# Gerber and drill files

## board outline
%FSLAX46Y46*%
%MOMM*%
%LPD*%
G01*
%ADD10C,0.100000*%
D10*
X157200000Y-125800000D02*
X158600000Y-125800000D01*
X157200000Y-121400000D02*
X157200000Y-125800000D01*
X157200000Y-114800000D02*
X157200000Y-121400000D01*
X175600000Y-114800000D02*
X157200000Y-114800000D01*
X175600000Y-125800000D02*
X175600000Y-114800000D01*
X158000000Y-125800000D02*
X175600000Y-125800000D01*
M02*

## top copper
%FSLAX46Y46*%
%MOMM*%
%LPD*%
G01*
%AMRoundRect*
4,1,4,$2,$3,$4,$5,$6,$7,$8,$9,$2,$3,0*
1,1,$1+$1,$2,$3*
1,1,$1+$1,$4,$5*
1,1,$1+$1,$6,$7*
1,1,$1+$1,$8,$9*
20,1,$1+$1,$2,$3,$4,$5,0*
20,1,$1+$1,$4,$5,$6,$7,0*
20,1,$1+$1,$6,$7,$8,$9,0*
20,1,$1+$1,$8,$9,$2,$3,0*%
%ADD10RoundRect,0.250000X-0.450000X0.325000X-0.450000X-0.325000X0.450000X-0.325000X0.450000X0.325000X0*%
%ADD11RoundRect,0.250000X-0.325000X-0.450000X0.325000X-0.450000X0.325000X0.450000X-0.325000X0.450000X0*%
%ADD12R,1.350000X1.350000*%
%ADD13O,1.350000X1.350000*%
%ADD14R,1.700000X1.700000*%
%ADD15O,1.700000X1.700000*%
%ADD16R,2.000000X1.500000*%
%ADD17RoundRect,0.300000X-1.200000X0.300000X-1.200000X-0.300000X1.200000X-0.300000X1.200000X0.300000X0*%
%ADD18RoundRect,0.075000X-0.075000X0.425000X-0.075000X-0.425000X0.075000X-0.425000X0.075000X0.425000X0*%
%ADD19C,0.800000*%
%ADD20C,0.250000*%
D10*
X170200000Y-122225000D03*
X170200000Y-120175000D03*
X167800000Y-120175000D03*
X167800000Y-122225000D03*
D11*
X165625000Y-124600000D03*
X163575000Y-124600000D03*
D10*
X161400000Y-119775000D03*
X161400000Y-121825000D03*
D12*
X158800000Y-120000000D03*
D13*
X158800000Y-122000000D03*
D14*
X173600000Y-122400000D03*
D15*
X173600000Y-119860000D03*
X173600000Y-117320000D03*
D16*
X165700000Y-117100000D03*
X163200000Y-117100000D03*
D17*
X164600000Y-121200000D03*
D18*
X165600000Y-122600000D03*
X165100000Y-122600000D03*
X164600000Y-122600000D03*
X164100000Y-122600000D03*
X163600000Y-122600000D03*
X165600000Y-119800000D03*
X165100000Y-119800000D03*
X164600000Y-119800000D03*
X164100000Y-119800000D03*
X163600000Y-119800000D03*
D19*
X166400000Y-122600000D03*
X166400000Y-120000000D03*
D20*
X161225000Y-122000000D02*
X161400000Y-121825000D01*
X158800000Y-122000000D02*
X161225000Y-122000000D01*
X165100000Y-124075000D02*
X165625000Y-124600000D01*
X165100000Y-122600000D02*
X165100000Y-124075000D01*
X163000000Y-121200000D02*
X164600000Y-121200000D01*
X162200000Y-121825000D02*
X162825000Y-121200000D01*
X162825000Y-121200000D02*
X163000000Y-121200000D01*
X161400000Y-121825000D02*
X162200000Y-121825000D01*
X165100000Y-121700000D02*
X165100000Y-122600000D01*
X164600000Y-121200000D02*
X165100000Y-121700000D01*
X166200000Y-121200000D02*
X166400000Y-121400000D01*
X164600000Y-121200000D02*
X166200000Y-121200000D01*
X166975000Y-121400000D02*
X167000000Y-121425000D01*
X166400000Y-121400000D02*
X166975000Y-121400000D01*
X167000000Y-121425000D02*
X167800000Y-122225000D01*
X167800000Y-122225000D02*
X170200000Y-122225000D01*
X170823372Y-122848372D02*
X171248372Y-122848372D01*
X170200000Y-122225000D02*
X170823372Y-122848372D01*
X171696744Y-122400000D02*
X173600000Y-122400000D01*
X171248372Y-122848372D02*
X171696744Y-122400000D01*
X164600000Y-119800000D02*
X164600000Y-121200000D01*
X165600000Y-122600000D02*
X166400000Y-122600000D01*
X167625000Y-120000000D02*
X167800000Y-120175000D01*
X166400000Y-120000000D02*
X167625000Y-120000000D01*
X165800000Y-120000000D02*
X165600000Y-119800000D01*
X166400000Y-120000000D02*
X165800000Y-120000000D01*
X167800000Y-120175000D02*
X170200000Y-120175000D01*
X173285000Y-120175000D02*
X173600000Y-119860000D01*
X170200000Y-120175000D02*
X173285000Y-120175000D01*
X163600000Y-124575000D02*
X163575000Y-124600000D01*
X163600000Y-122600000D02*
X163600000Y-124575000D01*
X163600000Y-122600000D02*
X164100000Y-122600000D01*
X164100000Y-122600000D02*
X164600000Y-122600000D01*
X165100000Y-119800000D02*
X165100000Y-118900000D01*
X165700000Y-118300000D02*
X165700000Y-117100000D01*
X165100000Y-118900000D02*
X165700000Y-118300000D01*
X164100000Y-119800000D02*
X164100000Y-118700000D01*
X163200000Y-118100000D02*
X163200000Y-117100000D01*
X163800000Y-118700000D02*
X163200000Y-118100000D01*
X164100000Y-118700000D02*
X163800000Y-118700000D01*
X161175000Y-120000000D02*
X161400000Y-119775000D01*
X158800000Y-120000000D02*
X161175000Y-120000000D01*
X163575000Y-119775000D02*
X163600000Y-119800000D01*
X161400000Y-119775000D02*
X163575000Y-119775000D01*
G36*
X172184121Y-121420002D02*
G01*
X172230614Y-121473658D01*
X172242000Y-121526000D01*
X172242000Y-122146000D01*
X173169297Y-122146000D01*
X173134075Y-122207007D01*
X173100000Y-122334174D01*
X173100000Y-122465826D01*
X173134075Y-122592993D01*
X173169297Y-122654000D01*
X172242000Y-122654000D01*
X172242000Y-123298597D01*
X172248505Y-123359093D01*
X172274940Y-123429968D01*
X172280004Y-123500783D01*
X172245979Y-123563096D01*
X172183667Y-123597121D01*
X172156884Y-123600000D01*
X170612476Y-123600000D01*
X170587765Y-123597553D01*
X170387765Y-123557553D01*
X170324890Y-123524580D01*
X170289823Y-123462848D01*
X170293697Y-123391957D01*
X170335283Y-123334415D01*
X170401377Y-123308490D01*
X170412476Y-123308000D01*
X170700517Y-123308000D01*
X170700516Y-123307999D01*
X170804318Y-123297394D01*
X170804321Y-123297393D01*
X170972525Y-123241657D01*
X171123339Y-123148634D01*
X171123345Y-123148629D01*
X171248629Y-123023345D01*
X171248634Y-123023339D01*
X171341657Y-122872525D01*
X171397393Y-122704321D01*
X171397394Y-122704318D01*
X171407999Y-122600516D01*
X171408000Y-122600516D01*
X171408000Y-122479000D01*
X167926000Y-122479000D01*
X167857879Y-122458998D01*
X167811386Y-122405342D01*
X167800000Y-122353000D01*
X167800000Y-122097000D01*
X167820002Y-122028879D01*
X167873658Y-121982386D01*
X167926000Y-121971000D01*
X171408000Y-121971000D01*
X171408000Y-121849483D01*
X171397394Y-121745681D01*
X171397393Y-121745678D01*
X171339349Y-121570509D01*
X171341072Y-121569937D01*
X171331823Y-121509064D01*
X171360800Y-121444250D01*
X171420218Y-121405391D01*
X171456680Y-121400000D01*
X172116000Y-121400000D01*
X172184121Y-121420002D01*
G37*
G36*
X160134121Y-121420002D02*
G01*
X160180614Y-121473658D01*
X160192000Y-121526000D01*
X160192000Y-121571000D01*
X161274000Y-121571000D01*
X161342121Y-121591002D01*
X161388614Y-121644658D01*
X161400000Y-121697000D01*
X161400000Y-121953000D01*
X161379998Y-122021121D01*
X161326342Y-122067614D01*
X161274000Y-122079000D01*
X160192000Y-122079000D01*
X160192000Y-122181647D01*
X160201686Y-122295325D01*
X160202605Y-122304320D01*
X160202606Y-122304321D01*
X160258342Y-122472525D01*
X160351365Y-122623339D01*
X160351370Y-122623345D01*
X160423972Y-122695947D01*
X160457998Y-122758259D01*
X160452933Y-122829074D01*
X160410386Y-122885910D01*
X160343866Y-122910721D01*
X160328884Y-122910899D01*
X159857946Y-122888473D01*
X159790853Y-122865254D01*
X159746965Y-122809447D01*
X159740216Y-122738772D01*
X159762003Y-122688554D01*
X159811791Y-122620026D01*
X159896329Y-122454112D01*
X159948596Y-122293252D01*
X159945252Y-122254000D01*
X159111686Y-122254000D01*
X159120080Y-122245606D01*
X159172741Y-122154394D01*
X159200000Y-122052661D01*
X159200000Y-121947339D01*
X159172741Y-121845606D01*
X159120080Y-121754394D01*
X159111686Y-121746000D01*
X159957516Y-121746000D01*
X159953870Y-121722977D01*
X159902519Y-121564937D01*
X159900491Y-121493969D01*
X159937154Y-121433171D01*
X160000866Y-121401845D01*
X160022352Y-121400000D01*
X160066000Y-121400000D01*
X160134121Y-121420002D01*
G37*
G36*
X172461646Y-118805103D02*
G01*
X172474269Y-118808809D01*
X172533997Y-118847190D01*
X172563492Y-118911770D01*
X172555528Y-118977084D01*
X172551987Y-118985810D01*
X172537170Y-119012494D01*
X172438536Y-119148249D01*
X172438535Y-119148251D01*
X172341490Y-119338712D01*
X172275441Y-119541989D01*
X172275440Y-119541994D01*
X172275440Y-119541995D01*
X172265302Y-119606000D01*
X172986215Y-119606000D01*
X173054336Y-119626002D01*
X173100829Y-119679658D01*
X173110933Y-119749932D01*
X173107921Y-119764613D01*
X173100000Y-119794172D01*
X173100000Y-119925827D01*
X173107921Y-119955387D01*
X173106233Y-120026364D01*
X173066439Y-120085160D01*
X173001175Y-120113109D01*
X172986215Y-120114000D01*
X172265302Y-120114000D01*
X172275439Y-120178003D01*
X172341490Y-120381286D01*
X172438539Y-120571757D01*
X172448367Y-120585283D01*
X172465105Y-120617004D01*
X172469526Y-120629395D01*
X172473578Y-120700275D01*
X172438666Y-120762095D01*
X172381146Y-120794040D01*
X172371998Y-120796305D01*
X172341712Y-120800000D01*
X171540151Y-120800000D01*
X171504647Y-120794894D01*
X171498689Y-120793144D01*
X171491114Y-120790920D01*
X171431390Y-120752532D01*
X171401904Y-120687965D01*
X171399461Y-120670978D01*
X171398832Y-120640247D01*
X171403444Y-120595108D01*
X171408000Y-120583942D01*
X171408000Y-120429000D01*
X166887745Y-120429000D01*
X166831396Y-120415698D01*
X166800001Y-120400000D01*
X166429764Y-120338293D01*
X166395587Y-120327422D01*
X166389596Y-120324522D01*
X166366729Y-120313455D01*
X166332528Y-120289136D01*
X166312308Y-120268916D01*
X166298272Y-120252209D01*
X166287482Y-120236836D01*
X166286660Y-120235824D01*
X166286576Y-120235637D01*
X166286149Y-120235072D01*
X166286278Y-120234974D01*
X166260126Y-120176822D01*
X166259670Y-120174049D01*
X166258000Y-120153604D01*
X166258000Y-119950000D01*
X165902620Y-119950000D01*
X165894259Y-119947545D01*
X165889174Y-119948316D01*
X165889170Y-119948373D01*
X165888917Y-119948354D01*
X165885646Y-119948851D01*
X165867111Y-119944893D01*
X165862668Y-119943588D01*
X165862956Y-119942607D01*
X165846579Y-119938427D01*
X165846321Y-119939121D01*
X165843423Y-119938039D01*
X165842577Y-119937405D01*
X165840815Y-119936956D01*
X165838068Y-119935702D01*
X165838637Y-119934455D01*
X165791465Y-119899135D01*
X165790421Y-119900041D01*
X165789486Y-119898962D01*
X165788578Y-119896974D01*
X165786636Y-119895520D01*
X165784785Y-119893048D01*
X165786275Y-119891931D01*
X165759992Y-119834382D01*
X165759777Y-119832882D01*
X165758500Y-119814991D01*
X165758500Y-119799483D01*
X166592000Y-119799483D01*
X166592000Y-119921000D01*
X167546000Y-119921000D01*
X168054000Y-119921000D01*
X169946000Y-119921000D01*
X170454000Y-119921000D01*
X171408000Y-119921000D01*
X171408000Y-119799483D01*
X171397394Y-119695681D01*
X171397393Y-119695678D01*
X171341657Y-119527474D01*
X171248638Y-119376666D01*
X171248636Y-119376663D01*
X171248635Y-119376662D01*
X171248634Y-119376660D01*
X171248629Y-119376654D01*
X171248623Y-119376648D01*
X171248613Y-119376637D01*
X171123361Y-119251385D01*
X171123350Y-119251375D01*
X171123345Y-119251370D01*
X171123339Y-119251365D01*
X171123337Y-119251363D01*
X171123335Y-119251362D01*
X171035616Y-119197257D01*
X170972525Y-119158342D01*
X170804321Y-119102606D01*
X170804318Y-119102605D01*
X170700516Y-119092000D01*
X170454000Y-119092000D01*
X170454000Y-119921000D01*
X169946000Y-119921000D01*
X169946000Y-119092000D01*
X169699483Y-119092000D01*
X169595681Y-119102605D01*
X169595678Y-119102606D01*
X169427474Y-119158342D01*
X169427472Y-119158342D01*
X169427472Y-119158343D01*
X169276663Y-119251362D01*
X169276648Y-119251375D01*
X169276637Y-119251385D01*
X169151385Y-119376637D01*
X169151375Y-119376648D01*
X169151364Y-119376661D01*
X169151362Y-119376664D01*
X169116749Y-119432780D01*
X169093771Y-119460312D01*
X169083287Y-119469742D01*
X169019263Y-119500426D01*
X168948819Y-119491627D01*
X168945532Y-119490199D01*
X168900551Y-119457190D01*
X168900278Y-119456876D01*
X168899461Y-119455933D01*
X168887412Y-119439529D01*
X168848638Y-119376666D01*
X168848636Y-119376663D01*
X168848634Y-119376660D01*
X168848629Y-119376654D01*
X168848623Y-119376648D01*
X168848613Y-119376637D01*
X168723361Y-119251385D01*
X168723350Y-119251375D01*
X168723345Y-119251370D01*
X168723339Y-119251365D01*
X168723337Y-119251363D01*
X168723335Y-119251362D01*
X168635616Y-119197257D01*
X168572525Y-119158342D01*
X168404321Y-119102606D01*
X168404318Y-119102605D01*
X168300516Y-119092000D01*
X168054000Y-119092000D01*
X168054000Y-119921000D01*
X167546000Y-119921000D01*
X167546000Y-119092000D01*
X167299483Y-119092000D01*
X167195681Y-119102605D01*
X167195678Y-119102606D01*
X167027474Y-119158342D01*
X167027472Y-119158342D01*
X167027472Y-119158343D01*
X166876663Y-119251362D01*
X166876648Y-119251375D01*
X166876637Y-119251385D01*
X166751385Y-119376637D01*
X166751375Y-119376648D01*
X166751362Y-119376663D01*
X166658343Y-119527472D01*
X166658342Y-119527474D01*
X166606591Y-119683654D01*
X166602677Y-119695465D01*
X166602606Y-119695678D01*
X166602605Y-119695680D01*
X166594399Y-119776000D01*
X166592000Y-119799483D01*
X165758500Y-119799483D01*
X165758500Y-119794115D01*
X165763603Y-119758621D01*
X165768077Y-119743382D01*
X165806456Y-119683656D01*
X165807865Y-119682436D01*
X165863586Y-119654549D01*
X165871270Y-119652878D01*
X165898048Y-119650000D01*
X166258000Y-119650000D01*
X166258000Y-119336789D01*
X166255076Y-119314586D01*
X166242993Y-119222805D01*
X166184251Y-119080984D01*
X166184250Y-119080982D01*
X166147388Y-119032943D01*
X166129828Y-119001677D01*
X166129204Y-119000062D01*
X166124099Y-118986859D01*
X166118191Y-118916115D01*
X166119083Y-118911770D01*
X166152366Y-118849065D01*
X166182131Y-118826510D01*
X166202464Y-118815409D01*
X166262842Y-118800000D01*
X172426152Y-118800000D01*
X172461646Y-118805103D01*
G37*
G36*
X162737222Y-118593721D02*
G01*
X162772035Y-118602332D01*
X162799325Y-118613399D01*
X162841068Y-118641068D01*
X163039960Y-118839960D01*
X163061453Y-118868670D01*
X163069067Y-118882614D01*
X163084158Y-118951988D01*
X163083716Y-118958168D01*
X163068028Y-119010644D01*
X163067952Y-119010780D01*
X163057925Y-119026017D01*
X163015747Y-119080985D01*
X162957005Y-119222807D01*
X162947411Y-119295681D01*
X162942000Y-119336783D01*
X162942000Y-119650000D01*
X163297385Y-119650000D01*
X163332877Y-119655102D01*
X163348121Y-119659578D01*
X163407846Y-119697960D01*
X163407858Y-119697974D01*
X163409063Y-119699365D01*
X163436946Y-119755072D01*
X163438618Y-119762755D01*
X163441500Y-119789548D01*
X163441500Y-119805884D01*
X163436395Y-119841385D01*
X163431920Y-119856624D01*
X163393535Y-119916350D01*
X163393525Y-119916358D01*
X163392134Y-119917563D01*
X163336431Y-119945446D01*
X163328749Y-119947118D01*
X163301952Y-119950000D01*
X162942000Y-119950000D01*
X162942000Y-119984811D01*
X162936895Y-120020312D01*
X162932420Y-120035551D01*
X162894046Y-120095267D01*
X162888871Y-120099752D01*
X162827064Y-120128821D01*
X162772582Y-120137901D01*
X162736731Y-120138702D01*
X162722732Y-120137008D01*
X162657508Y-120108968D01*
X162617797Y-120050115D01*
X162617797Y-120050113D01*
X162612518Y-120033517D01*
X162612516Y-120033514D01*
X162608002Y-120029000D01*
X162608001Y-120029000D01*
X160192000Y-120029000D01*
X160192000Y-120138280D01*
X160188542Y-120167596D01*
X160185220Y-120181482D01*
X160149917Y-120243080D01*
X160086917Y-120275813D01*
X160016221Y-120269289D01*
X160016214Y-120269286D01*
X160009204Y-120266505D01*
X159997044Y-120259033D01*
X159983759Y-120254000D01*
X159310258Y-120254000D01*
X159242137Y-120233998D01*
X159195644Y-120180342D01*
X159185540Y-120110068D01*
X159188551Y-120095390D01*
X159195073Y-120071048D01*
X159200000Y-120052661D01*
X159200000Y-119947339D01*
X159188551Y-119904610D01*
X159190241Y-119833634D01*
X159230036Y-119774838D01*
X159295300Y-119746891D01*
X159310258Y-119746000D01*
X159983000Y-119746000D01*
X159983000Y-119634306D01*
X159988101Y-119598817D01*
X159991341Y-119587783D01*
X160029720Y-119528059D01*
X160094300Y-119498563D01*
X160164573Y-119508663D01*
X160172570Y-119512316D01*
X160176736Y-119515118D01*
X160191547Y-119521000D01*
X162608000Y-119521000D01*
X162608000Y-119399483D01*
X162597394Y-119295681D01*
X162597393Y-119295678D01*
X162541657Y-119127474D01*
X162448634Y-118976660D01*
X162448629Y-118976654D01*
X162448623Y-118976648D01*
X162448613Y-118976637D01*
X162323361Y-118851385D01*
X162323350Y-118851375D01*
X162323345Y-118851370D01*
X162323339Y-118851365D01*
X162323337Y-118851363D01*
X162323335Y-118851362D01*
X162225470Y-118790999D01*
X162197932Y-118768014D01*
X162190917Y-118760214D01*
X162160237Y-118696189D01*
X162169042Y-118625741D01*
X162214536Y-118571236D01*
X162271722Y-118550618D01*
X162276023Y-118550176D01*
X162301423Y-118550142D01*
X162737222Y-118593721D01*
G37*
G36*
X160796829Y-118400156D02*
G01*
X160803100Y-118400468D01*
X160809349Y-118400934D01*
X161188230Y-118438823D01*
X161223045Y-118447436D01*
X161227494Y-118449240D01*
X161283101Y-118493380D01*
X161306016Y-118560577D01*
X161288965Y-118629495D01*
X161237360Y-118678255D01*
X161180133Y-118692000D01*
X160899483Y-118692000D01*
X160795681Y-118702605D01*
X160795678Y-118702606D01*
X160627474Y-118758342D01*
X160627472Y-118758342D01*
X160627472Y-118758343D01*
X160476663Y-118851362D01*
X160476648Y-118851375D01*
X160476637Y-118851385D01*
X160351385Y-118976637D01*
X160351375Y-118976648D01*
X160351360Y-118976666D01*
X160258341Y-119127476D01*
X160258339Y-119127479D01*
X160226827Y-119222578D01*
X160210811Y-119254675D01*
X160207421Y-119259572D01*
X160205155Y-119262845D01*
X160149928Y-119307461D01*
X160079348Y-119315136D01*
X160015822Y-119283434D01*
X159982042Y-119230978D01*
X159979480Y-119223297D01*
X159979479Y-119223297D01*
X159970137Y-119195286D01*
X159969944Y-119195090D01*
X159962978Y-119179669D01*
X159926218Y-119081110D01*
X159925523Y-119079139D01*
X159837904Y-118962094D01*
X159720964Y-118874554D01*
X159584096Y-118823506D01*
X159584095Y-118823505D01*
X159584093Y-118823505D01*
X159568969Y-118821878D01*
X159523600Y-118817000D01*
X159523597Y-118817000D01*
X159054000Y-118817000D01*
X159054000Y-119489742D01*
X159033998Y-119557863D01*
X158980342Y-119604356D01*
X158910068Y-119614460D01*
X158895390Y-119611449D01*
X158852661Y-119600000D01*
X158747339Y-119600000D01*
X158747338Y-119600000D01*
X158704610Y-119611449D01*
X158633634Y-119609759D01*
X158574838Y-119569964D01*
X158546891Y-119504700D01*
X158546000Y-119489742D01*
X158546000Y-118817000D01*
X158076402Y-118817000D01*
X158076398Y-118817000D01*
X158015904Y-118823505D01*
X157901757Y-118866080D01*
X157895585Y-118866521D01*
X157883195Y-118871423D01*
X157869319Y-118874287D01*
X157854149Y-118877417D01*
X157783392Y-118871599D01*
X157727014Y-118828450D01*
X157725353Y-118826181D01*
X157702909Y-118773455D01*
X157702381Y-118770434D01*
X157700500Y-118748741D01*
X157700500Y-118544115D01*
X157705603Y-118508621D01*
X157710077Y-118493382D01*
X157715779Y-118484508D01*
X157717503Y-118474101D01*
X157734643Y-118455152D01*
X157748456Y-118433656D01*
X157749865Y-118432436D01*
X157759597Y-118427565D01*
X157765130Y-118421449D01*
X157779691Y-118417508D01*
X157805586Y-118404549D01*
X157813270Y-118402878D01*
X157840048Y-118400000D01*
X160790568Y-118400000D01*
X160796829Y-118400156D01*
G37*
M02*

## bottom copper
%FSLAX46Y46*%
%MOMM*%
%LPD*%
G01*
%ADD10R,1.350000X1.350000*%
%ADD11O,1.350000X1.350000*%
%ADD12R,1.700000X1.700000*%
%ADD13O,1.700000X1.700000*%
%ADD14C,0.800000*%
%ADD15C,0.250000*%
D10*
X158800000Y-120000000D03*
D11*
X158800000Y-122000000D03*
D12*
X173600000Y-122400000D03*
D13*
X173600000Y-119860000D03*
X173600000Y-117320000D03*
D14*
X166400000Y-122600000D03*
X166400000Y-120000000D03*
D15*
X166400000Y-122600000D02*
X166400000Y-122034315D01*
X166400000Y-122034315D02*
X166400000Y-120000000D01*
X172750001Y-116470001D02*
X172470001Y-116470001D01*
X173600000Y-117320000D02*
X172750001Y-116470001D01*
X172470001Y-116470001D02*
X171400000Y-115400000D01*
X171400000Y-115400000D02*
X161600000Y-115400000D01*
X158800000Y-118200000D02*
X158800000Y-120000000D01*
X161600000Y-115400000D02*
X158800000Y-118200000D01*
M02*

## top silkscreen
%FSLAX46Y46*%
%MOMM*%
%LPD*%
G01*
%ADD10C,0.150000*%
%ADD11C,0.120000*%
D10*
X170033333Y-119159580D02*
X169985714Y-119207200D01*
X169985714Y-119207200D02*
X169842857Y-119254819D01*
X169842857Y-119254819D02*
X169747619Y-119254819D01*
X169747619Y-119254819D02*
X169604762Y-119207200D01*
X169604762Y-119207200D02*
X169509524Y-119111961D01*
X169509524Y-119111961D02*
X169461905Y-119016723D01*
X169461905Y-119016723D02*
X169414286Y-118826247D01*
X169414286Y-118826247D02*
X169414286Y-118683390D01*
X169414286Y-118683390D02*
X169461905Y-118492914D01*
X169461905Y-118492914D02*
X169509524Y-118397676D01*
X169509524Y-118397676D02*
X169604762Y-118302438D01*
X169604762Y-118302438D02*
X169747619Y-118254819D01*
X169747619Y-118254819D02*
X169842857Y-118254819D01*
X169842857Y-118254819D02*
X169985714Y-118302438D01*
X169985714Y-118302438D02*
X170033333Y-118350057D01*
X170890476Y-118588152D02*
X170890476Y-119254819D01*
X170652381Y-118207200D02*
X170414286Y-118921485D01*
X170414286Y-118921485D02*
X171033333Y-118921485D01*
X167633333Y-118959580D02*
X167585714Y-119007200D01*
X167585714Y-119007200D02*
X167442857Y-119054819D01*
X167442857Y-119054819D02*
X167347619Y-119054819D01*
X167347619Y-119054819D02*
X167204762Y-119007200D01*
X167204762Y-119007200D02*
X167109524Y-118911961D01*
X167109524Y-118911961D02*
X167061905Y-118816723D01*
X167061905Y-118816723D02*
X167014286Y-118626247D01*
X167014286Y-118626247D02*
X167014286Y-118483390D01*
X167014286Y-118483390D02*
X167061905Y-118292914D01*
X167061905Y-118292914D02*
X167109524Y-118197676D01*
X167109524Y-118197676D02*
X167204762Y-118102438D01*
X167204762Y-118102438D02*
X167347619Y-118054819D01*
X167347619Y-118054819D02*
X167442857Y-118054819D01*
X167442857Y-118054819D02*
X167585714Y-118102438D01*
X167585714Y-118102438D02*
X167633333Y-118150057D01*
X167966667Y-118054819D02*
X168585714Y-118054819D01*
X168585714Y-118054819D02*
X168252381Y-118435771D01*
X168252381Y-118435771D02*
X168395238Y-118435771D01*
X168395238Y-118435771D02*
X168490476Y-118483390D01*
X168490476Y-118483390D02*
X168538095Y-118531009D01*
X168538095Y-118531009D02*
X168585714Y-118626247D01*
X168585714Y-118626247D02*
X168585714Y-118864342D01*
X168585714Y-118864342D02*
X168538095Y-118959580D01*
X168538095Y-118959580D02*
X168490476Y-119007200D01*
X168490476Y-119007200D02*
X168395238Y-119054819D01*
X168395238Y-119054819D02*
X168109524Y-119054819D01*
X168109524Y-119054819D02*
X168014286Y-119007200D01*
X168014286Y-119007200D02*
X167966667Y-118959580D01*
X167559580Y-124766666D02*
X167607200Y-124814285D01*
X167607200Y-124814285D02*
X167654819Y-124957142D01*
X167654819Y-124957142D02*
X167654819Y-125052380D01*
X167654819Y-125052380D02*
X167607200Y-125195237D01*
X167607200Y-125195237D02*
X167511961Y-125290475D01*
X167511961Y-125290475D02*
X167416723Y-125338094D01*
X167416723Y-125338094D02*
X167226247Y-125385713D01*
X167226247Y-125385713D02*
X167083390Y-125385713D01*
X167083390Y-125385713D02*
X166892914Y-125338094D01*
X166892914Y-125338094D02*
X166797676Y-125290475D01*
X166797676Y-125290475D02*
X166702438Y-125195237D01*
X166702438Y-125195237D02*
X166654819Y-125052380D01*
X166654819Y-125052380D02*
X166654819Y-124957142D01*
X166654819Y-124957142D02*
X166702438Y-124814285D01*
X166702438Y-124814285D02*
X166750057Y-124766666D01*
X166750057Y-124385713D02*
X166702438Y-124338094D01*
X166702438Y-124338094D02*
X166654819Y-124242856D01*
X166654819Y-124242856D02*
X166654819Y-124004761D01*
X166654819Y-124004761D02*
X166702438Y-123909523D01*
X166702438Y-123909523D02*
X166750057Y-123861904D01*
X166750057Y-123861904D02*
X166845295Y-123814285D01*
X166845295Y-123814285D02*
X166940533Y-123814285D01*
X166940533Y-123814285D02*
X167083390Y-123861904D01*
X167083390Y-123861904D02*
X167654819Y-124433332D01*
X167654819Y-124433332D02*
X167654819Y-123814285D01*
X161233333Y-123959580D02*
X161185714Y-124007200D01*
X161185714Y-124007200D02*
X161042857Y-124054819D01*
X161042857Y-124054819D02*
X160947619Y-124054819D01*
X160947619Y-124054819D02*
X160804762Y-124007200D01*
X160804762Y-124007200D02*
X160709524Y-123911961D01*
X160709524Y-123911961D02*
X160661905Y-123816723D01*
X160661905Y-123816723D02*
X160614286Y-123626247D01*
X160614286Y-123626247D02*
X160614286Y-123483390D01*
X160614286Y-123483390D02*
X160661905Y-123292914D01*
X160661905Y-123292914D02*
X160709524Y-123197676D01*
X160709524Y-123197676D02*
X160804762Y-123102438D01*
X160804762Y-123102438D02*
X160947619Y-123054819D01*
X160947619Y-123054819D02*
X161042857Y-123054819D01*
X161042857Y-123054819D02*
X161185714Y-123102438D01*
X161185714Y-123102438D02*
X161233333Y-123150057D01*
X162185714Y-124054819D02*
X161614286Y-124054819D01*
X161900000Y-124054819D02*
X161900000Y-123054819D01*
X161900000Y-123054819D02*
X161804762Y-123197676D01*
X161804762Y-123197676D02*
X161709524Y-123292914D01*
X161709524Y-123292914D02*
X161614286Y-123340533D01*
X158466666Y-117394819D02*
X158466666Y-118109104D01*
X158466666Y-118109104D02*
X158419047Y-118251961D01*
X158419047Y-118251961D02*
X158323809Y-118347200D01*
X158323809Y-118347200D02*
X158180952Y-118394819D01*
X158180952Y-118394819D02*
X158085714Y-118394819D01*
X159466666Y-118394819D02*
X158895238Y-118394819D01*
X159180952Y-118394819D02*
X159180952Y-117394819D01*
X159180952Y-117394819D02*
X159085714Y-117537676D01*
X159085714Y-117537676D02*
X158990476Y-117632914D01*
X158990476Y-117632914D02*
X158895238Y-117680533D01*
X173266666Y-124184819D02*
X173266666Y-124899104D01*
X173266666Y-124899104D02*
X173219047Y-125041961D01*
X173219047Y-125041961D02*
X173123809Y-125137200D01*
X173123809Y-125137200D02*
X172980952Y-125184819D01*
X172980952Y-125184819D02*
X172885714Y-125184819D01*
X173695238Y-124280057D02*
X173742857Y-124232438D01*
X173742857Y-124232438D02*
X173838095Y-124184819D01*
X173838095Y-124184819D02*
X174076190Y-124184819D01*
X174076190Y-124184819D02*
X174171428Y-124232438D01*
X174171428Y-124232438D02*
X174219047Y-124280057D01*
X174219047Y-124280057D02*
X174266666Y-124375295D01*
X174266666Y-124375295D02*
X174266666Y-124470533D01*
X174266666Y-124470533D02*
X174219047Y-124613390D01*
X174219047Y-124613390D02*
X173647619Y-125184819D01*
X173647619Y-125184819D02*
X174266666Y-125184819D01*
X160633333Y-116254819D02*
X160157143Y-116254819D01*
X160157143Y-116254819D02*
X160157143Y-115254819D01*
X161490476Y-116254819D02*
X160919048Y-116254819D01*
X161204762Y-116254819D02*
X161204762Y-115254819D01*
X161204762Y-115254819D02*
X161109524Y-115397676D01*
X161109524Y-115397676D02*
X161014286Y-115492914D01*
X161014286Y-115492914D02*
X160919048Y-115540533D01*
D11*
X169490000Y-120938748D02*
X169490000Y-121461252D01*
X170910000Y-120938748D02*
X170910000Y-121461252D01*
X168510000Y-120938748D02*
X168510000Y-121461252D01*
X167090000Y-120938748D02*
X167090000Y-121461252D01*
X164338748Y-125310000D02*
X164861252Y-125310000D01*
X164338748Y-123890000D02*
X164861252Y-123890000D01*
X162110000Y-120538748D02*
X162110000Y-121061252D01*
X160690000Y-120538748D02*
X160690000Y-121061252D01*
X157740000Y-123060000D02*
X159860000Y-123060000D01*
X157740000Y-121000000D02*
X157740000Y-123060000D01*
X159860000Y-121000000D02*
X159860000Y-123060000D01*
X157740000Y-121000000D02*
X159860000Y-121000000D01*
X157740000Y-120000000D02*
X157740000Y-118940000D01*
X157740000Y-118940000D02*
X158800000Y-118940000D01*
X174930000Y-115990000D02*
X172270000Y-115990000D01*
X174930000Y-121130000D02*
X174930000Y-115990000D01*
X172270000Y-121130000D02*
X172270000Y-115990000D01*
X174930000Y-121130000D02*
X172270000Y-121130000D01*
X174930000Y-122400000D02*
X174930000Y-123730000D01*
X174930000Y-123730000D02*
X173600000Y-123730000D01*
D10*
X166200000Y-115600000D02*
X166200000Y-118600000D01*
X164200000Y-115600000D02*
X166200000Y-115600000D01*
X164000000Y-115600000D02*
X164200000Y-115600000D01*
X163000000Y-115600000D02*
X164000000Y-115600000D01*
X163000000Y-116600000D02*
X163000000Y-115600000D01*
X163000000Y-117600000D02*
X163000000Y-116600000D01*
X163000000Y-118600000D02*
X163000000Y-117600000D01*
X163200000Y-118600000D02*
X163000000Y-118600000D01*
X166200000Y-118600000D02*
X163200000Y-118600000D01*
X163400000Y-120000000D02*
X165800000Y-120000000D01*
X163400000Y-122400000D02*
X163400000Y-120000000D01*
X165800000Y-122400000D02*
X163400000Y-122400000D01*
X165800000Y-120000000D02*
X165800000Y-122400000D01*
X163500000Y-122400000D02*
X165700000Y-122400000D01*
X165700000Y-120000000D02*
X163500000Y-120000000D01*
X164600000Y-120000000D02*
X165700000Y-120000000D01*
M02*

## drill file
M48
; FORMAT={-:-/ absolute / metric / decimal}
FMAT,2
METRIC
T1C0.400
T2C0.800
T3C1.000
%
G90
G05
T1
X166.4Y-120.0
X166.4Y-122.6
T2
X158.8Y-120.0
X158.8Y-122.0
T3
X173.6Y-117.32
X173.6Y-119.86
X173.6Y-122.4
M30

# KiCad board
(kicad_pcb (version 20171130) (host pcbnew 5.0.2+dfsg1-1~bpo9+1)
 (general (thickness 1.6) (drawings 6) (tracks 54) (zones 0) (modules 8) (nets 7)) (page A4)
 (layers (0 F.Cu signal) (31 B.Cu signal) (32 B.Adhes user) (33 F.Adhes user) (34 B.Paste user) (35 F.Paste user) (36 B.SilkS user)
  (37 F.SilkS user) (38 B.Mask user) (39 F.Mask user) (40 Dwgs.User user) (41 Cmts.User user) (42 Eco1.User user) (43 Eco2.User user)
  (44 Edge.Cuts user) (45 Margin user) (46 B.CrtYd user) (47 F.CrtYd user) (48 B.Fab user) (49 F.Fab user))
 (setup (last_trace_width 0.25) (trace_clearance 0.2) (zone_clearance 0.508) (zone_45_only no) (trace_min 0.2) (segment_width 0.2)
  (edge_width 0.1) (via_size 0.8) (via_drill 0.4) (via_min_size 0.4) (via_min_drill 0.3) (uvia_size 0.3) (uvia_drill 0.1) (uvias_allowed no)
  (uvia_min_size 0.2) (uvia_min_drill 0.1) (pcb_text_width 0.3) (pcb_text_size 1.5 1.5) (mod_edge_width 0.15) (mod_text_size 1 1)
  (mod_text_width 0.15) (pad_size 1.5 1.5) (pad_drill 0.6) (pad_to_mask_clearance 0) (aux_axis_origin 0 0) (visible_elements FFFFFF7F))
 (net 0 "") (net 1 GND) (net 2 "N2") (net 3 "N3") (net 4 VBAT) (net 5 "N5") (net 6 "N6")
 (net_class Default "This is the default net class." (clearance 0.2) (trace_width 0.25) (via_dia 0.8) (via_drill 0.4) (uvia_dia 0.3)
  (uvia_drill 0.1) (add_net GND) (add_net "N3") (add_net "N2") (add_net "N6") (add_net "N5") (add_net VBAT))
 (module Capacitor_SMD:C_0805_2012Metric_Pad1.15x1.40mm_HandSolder (layer F.Cu) (at 170.2 121.2 270)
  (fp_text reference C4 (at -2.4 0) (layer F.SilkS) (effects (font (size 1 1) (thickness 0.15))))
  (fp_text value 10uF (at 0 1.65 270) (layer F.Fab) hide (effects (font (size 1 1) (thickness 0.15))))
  (fp_line (start -0.261252 0.71) (end 0.261252 0.71) (layer F.SilkS) (width 0.12))
  (fp_line (start -0.261252 -0.71) (end 0.261252 -0.71) (layer F.SilkS) (width 0.12))
  (pad 2 smd roundrect (at 1.025 0 270) (size 1.15 1.4) (layers F.Cu F.Paste F.Mask) (roundrect_rratio 0.217391) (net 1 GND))
  (pad 1 smd roundrect (at -1.025 0 270) (size 1.15 1.4) (layers F.Cu F.Paste F.Mask) (roundrect_rratio 0.217391) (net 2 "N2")))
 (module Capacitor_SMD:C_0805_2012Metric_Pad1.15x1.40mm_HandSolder (layer F.Cu) (at 167.8 121.2 270)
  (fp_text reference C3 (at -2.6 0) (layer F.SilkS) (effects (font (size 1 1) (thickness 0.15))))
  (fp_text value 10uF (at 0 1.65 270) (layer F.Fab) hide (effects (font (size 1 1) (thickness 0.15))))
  (fp_line (start -0.261252 -0.71) (end 0.261252 -0.71) (layer F.SilkS) (width 0.12))
  (fp_line (start -0.261252 0.71) (end 0.261252 0.71) (layer F.SilkS) (width 0.12))
  (pad 1 smd roundrect (at -1.025 0 270) (size 1.15 1.4) (layers F.Cu F.Paste F.Mask) (roundrect_rratio 0.217391) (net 2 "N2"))
  (pad 2 smd roundrect (at 1.025 0 270) (size 1.15 1.4) (layers F.Cu F.Paste F.Mask) (roundrect_rratio 0.217391) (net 1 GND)))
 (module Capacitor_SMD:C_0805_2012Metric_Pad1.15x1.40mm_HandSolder (layer F.Cu) (at 164.6 124.6)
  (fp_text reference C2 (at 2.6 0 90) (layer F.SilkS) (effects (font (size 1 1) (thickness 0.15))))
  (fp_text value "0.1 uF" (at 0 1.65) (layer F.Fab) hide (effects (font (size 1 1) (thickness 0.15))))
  (fp_line (start -0.261252 0.71) (end 0.261252 0.71) (layer F.SilkS) (width 0.12))
  (fp_line (start -0.261252 -0.71) (end 0.261252 -0.71) (layer F.SilkS) (width 0.12))
  (pad 2 smd roundrect (at 1.025 0) (size 1.15 1.4) (layers F.Cu F.Paste F.Mask) (roundrect_rratio 0.217391) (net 1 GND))
  (pad 1 smd roundrect (at -1.025 0) (size 1.15 1.4) (layers F.Cu F.Paste F.Mask) (roundrect_rratio 0.217391) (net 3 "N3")))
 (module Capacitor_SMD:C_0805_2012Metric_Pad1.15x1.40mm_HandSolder (layer F.Cu) (at 161.4 120.8 270)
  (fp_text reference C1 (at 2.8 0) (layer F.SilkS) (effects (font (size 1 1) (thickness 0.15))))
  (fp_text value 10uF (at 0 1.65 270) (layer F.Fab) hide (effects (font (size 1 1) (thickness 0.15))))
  (fp_line (start -0.261252 -0.71) (end 0.261252 -0.71) (layer F.SilkS) (width 0.12))
  (fp_line (start -0.261252 0.71) (end 0.261252 0.71) (layer F.SilkS) (width 0.12))
  (pad 1 smd roundrect (at -1.025 0 270) (size 1.15 1.4) (layers F.Cu F.Paste F.Mask) (roundrect_rratio 0.217391) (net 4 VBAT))
  (pad 2 smd roundrect (at 1.025 0 270) (size 1.15 1.4) (layers F.Cu F.Paste F.Mask) (roundrect_rratio 0.217391) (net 1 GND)))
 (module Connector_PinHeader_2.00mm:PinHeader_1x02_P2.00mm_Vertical (layer F.Cu) (at 158.8 120)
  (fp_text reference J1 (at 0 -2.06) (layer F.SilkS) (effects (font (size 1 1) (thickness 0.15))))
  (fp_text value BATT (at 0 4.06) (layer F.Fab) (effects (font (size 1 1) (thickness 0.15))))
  (fp_line (start -1.06 3.06) (end 1.06 3.06) (layer F.SilkS) (width 0.12))
  (fp_line (start -1.06 1) (end -1.06 3.06) (layer F.SilkS) (width 0.12))
  (fp_line (start 1.06 1) (end 1.06 3.06) (layer F.SilkS) (width 0.12))
  (fp_line (start -1.06 1) (end 1.06 1) (layer F.SilkS) (width 0.12))
  (fp_line (start -1.06 0) (end -1.06 -1.06) (layer F.SilkS) (width 0.12))
  (fp_line (start -1.06 -1.06) (end 0 -1.06) (layer F.SilkS) (width 0.12))
  (pad 1 thru_hole rect (at 0 0) (size 1.35 1.35) (drill 0.8) (layers *.Cu *.Mask) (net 4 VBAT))
  (pad 2 thru_hole oval (at 0 2) (size 1.35 1.35) (drill 0.8) (layers *.Cu *.Mask) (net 1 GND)))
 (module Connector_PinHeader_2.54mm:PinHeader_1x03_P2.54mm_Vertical (layer F.Cu) (at 173.6 122.4 180)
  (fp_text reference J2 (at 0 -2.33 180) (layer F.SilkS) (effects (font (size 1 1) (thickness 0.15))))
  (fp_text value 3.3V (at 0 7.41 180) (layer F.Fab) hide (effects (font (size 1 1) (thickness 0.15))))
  (fp_line (start -1.33 6.41) (end 1.33 6.41) (layer F.SilkS) (width 0.12))
  (fp_line (start -1.33 1.27) (end -1.33 6.41) (layer F.SilkS) (width 0.12))
  (fp_line (start 1.33 1.27) (end 1.33 6.41) (layer F.SilkS) (width 0.12))
  (fp_line (start -1.33 1.27) (end 1.33 1.27) (layer F.SilkS) (width 0.12))
  (fp_line (start -1.33 0) (end -1.33 -1.33) (layer F.SilkS) (width 0.12))
  (fp_line (start -1.33 -1.33) (end 0 -1.33) (layer F.SilkS) (width 0.12))
  (pad 1 thru_hole rect (at 0 0 180) (size 1.7 1.7) (drill 1) (layers *.Cu *.Mask) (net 1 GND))
  (pad 2 thru_hole oval (at 0 2.54 180) (size 1.7 1.7) (drill 1) (layers *.Cu *.Mask) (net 2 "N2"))
  (pad 3 thru_hole oval (at 0 5.08 180) (size 1.7 1.7) (drill 1) (layers *.Cu *.Mask) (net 4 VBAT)))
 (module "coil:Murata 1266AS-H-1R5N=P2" (layer F.Cu) (at 164.2 116.6 180)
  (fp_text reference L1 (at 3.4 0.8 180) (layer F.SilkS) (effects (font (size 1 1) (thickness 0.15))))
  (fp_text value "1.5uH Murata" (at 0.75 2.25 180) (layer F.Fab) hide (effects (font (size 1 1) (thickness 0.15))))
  (fp_line (start -2 1) (end -2 -2) (layer F.SilkS) (width 0.15))
  (fp_line (start 0 1) (end -2 1) (layer F.SilkS) (width 0.15))
  (fp_line (start 0.2 1) (end 0 1) (layer F.SilkS) (width 0.15))
  (fp_line (start 1.2 1) (end 0.2 1) (layer F.SilkS) (width 0.15))
  (fp_line (start 1.2 0) (end 1.2 1) (layer F.SilkS) (width 0.15))
  (fp_line (start 1.2 -1) (end 1.2 0) (layer F.SilkS) (width 0.15))
  (fp_line (start 1.2 -2) (end 1.2 -1) (layer F.SilkS) (width 0.15))
  (fp_line (start 1 -2) (end 1.2 -2) (layer F.SilkS) (width 0.15))
  (fp_line (start -2 -2) (end 1 -2) (layer F.SilkS) (width 0.15))
  (pad 2 smd rect (at -1.5 -0.5 180) (size 2 1.5) (layers F.Cu F.Paste F.Mask) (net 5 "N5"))
  (pad 1 smd rect (at 1 -0.5 180) (size 2 1.5) (layers F.Cu F.Paste F.Mask) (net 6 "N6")))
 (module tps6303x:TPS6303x (layer F.Cu) (at 164.6 121.2 270)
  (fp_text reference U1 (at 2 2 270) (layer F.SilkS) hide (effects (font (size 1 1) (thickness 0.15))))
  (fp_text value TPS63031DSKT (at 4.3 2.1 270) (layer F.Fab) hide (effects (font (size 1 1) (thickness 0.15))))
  (fp_line (start -1.2 1.2) (end -1.2 -1.2) (layer F.SilkS) (width 0.15))
  (fp_line (start 1.2 1.2) (end -1.2 1.2) (layer F.SilkS) (width 0.15))
  (fp_line (start 1.2 -1.2) (end 1.2 1.2) (layer F.SilkS) (width 0.15))
  (fp_line (start -1.2 -1.2) (end 1.2 -1.2) (layer F.SilkS) (width 0.15))
  (fp_line (start 1.2 1.1) (end 1.2 -1.1) (layer F.SilkS) (width 0.15))
  (fp_line (start -1.2 -1.1) (end -1.2 1.1) (layer F.SilkS) (width 0.15))
  (fp_line (start -1.2 0) (end -1.2 -1.1) (layer F.SilkS) (width 0.15))
  (pad 3 smd roundrect (at 0 0 270) (size 1.2 3) (layers F.Cu F.Paste F.Mask) (roundrect_rratio 0.25) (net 1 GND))
  (pad 10 smd roundrect (at 1.4 -1 270) (size 1 0.3) (layers F.Cu F.Paste F.Mask) (roundrect_rratio 0.25) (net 2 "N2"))
  (pad 9 smd roundrect (at 1.4 -0.5 270) (size 1 0.3) (layers F.Cu F.Paste F.Mask) (roundrect_rratio 0.25) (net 1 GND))
  (pad 8 smd roundrect (at 1.4 0 270) (size 1 0.3) (layers F.Cu F.Paste F.Mask) (roundrect_rratio 0.25) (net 3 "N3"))
  (pad 7 smd roundrect (at 1.4 0.5 270) (size 1 0.3) (layers F.Cu F.Paste F.Mask) (roundrect_rratio 0.25) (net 3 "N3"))
  (pad 6 smd roundrect (at 1.4 1 270) (size 1 0.3) (layers F.Cu F.Paste F.Mask) (roundrect_rratio 0.25) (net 3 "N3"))
  (pad 1 smd roundrect (at -1.4 -1 270) (size 1 0.3) (layers F.Cu F.Paste F.Mask) (roundrect_rratio 0.25) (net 2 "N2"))
  (pad 2 smd roundrect (at -1.4 -0.5 270) (size 1 0.3) (layers F.Cu F.Paste F.Mask) (roundrect_rratio 0.25) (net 5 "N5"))
  (pad 3 smd roundrect (at -1.4 0 270) (size 1 0.3) (layers F.Cu F.Paste F.Mask) (roundrect_rratio 0.25) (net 1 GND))
  (pad 4 smd roundrect (at -1.4 0.5 270) (size 1 0.3) (layers F.Cu F.Paste F.Mask) (roundrect_rratio 0.25) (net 6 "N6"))
  (pad 5 smd roundrect (at -1.4 1 270) (size 1 0.3) (layers F.Cu F.Paste F.Mask) (roundrect_rratio 0.25) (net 4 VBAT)))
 (gr_line (start 157.2 125.8) (end 158.6 125.8) (layer Edge.Cuts) (width 0.1))
 (gr_line (start 157.2 121.4) (end 157.2 125.8) (layer Edge.Cuts) (width 0.1))
 (gr_line (start 157.2 114.8) (end 157.2 121.4) (layer Edge.Cuts) (width 0.1))
 (gr_line (start 175.6 114.8) (end 157.2 114.8) (layer Edge.Cuts) (width 0.1))
 (gr_line (start 175.6 125.8) (end 175.6 114.8) (layer Edge.Cuts) (width 0.1))
 (gr_line (start 158 125.8) (end 175.6 125.8) (layer Edge.Cuts) (width 0.1))
 (segment (start 161.225 122) (end 161.4 121.825) (width 0.25) (layer F.Cu) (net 1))
 (segment (start 158.8 122) (end 161.225 122) (width 0.25) (layer F.Cu) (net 1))
 (segment (start 165.1 124.075) (end 165.625 124.6) (width 0.25) (layer F.Cu) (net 1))
 (segment (start 165.1 122.6) (end 165.1 124.075) (width 0.25) (layer F.Cu) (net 1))
 (segment (start 163 121.2) (end 164.6 121.2) (width 0.25) (layer F.Cu) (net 1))
 (segment (start 162.2 121.825) (end 162.825 121.2) (width 0.25) (layer F.Cu) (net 1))
 (segment (start 162.825 121.2) (end 163 121.2) (width 0.25) (layer F.Cu) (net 1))
 (segment (start 161.4 121.825) (end 162.2 121.825) (width 0.25) (layer F.Cu) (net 1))
 (segment (start 165.1 121.7) (end 165.1 122.6) (width 0.25) (layer F.Cu) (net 1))
 (segment (start 164.6 121.2) (end 165.1 121.7) (width 0.25) (layer F.Cu) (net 1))
 (segment (start 166.2 121.2) (end 166.4 121.4) (width 0.25) (layer F.Cu) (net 1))
 (segment (start 164.6 121.2) (end 166.2 121.2) (width 0.25) (layer F.Cu) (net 1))
 (segment (start 166.975 121.4) (end 167 121.425) (width 0.25) (layer F.Cu) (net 1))
 (segment (start 166.4 121.4) (end 166.975 121.4) (width 0.25) (layer F.Cu) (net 1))
 (segment (start 167 121.425) (end 167.8 122.225) (width 0.25) (layer F.Cu) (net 1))
 (segment (start 167.8 122.225) (end 170.2 122.225) (width 0.25) (layer F.Cu) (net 1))
 (segment (start 170.823372 122.848372) (end 171.248372 122.848372) (width 0.25) (layer F.Cu) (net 1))
 (segment (start 170.2 122.225) (end 170.823372 122.848372) (width 0.25) (layer F.Cu) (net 1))
 (segment (start 171.696744 122.4) (end 173.6 122.4) (width 0.25) (layer F.Cu) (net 1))
 (segment (start 171.248372 122.848372) (end 171.696744 122.4) (width 0.25) (layer F.Cu) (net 1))
 (segment (start 164.6 119.8) (end 164.6 121.2) (width 0.25) (layer F.Cu) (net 1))
 (segment (start 165.6 122.6) (end 166.4 122.6) (width 0.25) (layer F.Cu) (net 2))
 (via (at 166.4 122.6) (size 0.8) (drill 0.4) (layers F.Cu B.Cu) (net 2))
 (segment (start 166.4 122.6) (end 166.4 122.034315) (width 0.25) (layer B.Cu) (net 2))
 (via (at 166.4 120) (size 0.8) (drill 0.4) (layers F.Cu B.Cu) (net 2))
 (segment (start 166.4 122.034315) (end 166.4 120) (width 0.25) (layer B.Cu) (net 2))
 (segment (start 167.625 120) (end 167.8 120.175) (width 0.25) (layer F.Cu) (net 2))
 (segment (start 166.4 120) (end 167.625 120) (width 0.25) (layer F.Cu) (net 2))
 (segment (start 165.8 120) (end 165.6 119.8) (width 0.25) (layer F.Cu) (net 2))
 (segment (start 166.4 120) (end 165.8 120) (width 0.25) (layer F.Cu) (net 2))
 (segment (start 167.8 120.175) (end 170.2 120.175) (width 0.25) (layer F.Cu) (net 2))
 (segment (start 173.285 120.175) (end 173.6 119.86) (width 0.25) (layer F.Cu) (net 2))
 (segment (start 170.2 120.175) (end 173.285 120.175) (width 0.25) (layer F.Cu) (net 2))
 (segment (start 163.6 124.575) (end 163.575 124.6) (width 0.25) (layer F.Cu) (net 3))
 (segment (start 163.6 122.6) (end 163.6 124.575) (width 0.25) (layer F.Cu) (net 3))
 (segment (start 163.6 122.6) (end 164.1 122.6) (width 0.25) (layer F.Cu) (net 3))
 (segment (start 164.1 122.6) (end 164.6 122.6) (width 0.25) (layer F.Cu) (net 3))
 (segment (start 165.1 119.8) (end 165.1 118.9) (width 0.25) (layer F.Cu) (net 5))
 (segment (start 165.7 118.3) (end 165.7 117.1) (width 0.25) (layer F.Cu) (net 5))
 (segment (start 165.1 118.9) (end 165.7 118.3) (width 0.25) (layer F.Cu) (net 5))
 (segment (start 164.1 119.8) (end 164.1 118.7) (width 0.25) (layer F.Cu) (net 6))
 (segment (start 163.2 118.1) (end 163.2 117.1) (width 0.25) (layer F.Cu) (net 6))
 (segment (start 163.8 118.7) (end 163.2 118.1) (width 0.25) (layer F.Cu) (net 6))
 (segment (start 164.1 118.7) (end 163.8 118.7) (width 0.25) (layer F.Cu) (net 6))
 (segment (start 161.175 120) (end 161.4 119.775) (width 0.25) (layer F.Cu) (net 4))
 (segment (start 158.8 120) (end 161.175 120) (width 0.25) (layer F.Cu) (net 4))
 (segment (start 163.575 119.775) (end 163.6 119.8) (width 0.25) (layer F.Cu) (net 4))
 (segment (start 161.4 119.775) (end 163.575 119.775) (width 0.25) (layer F.Cu) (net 4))
 (segment (start 172.750001 116.470001) (end 172.470001 116.470001) (width 0.25) (layer B.Cu) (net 4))
 (segment (start 173.6 117.32) (end 172.750001 116.470001) (width 0.25) (layer B.Cu) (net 4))
 (segment (start 172.470001 116.470001) (end 171.4 115.4) (width 0.25) (layer B.Cu) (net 4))
 (segment (start 171.4 115.4) (end 161.6 115.4) (width 0.25) (layer B.Cu) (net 4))
 (segment (start 158.8 118.2) (end 158.8 120) (width 0.25) (layer B.Cu) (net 4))
 (segment (start 161.6 115.4) (end 158.8 118.2) (width 0.25) (layer B.Cu) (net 4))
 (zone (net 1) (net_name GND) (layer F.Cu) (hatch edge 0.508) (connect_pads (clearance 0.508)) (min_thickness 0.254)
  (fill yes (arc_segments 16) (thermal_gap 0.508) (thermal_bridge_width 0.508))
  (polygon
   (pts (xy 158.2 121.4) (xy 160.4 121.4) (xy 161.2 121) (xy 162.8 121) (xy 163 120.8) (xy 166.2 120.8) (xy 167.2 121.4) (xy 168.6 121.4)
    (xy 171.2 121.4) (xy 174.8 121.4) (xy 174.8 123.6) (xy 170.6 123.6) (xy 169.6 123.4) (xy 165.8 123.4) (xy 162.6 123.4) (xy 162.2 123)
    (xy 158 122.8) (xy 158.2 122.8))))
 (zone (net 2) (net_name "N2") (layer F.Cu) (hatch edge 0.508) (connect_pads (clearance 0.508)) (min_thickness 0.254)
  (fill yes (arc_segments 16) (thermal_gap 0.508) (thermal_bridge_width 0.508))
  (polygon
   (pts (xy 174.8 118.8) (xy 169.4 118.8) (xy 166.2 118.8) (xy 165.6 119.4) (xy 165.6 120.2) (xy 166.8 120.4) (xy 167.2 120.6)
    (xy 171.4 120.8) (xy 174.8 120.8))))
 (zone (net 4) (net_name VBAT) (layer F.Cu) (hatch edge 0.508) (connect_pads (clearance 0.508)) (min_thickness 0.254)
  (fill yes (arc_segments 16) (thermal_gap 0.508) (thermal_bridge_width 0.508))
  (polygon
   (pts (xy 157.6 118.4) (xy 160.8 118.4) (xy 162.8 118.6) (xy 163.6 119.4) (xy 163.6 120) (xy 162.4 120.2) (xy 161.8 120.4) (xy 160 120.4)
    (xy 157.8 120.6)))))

